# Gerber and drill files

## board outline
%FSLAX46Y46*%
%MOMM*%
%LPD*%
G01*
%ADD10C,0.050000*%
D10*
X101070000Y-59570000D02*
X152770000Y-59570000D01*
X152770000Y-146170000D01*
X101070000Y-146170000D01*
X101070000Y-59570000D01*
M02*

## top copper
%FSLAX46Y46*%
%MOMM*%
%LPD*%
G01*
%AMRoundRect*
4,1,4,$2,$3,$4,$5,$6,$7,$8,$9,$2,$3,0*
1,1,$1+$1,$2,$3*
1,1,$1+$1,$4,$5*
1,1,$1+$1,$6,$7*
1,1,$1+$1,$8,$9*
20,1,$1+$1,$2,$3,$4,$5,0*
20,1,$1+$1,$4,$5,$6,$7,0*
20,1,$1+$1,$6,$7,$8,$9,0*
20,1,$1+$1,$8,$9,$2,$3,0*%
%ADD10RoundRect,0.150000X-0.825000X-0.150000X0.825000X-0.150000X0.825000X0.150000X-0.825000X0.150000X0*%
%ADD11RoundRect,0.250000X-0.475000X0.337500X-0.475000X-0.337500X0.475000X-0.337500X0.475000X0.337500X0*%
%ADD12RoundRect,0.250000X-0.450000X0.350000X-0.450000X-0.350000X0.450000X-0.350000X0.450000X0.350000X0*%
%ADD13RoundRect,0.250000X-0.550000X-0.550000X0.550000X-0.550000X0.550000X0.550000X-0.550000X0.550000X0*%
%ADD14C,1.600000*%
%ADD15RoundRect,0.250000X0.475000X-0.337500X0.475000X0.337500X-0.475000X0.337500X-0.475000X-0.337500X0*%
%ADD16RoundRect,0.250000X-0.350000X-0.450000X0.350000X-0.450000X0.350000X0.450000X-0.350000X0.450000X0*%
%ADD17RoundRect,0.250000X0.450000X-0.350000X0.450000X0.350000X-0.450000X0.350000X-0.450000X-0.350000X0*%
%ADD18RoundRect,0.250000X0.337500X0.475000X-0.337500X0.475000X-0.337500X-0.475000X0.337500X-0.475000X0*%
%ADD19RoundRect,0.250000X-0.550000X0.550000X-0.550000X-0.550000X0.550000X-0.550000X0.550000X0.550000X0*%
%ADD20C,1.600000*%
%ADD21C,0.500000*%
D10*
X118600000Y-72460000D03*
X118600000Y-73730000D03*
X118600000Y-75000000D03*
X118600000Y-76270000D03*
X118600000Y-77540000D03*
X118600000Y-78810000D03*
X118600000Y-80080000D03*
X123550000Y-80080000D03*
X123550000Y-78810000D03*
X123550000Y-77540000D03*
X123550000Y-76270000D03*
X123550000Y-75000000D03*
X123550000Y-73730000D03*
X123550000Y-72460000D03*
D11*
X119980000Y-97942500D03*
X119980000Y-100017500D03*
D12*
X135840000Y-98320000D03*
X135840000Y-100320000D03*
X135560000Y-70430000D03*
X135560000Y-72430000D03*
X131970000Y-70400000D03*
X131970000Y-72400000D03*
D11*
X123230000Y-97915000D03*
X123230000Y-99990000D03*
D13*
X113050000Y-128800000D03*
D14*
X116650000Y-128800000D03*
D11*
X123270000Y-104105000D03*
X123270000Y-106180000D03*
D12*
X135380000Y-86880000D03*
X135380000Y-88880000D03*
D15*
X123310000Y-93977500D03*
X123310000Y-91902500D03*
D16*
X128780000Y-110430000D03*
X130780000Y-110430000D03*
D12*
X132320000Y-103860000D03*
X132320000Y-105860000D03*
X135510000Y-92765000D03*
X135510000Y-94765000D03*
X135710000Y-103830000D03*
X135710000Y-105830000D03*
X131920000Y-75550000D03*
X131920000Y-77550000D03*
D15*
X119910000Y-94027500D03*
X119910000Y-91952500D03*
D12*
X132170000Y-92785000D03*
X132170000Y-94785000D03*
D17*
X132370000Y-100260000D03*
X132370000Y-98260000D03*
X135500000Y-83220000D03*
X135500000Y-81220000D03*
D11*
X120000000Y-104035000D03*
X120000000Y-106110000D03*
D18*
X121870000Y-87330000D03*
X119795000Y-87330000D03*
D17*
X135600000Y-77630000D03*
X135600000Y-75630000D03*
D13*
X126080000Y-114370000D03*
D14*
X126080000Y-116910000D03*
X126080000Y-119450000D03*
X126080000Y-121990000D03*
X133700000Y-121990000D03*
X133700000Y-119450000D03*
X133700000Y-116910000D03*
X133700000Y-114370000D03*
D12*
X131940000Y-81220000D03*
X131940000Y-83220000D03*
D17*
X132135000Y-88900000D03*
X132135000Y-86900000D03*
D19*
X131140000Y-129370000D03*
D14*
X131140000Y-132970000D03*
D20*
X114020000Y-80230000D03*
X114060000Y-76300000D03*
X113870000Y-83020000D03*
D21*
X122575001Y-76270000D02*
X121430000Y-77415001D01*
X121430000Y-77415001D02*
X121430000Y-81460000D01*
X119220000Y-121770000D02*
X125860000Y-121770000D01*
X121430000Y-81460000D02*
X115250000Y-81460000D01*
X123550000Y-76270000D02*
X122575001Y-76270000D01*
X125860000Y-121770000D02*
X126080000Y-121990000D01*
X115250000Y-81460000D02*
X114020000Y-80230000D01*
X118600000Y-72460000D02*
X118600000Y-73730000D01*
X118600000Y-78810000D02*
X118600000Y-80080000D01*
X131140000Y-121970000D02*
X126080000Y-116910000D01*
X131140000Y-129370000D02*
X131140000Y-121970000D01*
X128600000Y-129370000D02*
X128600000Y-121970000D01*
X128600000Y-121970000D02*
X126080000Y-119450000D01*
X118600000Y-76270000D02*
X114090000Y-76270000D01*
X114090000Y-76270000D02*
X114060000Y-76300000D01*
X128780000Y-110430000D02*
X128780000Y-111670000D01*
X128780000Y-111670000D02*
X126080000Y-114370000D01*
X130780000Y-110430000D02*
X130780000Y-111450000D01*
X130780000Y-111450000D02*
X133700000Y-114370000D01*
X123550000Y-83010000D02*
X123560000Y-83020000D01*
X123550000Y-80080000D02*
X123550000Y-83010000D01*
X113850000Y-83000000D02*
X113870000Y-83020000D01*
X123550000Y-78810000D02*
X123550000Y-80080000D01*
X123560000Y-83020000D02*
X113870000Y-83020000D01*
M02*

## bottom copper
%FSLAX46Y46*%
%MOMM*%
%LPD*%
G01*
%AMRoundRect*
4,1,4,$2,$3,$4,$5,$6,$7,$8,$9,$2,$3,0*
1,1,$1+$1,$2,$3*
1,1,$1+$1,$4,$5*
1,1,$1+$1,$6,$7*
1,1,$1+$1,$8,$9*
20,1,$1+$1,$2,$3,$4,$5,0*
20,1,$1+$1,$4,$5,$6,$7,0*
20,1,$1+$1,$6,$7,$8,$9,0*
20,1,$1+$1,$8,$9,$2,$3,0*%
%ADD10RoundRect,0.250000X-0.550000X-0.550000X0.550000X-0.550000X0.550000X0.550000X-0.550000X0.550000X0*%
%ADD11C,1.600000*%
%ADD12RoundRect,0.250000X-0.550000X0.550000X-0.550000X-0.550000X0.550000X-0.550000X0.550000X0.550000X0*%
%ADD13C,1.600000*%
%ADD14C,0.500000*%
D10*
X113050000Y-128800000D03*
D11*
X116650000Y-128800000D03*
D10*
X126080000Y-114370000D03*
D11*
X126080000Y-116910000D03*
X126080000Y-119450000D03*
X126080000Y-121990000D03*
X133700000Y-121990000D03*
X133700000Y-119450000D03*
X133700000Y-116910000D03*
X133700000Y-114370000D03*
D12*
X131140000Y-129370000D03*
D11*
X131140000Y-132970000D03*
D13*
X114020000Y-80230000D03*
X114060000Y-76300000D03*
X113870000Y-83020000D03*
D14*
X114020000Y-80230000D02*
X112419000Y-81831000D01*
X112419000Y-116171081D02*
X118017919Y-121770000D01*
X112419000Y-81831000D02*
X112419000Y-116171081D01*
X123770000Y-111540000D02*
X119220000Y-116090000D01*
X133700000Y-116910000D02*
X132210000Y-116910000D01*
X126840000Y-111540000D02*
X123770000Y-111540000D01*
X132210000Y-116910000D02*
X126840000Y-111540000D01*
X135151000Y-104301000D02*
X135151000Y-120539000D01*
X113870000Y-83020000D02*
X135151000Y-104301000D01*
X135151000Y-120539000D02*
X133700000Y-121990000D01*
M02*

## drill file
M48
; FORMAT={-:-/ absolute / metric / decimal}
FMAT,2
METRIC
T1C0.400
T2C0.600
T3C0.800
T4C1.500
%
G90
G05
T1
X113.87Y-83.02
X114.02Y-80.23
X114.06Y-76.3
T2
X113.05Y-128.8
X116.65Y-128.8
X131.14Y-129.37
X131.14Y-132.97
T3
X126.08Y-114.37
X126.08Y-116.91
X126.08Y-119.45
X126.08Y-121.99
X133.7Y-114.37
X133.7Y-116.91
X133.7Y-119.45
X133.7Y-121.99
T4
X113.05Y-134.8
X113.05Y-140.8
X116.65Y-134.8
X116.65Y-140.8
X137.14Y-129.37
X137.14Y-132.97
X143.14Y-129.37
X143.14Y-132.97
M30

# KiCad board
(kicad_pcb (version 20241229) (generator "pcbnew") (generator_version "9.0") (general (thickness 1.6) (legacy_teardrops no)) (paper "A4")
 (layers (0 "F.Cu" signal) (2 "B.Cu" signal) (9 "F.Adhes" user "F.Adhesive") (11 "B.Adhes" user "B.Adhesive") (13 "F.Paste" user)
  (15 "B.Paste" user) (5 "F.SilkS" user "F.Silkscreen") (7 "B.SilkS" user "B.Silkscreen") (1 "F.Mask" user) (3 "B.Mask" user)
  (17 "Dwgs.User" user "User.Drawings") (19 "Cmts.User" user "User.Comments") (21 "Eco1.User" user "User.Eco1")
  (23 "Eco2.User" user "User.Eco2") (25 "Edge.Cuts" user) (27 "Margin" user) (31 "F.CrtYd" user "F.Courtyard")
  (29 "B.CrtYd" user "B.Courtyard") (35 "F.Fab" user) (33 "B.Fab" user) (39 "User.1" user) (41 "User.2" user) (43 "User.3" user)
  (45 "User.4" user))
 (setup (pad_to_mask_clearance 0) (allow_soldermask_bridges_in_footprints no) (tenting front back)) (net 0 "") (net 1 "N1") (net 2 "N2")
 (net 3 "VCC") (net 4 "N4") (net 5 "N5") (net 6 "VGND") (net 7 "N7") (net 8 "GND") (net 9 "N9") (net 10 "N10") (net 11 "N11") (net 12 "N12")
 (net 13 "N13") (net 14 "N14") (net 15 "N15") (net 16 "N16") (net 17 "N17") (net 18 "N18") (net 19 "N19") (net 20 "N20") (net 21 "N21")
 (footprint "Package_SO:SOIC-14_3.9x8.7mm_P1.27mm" (layer "F.Cu") (at 121.075 76.27)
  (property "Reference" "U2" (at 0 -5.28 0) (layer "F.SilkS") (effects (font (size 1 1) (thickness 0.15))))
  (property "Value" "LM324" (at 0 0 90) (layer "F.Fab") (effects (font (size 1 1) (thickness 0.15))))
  (pad "1" smd roundrect (at -2.475 -3.81) (size 1.95 0.6) (layers "F.Cu" "F.Mask" "F.Paste") (roundrect_rratio 0.25) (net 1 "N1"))
  (pad "2" smd roundrect (at -2.475 -2.54) (size 1.95 0.6) (layers "F.Cu" "F.Mask" "F.Paste") (roundrect_rratio 0.25) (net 1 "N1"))
  (pad "3" smd roundrect (at -2.475 -1.27) (size 1.95 0.6) (layers "F.Cu" "F.Mask" "F.Paste") (roundrect_rratio 0.25) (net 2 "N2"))
  (pad "4" smd roundrect (at -2.475 0) (size 1.95 0.6) (layers "F.Cu" "F.Mask" "F.Paste") (roundrect_rratio 0.25) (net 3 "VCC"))
  (pad "5" smd roundrect (at -2.475 1.27) (size 1.95 0.6) (layers "F.Cu" "F.Mask" "F.Paste") (roundrect_rratio 0.25) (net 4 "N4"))
  (pad "6" smd roundrect (at -2.475 2.54) (size 1.95 0.6) (layers "F.Cu" "F.Mask" "F.Paste") (roundrect_rratio 0.25) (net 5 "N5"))
  (pad "7" smd roundrect (at -2.475 3.81) (size 1.95 0.6) (layers "F.Cu" "F.Mask" "F.Paste") (roundrect_rratio 0.25) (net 5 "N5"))
  (pad "8" smd roundrect (at 2.475 3.81) (size 1.95 0.6) (layers "F.Cu" "F.Mask" "F.Paste") (roundrect_rratio 0.25) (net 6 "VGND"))
  (pad "9" smd roundrect (at 2.475 2.54) (size 1.95 0.6) (layers "F.Cu" "F.Mask" "F.Paste") (roundrect_rratio 0.25) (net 6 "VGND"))
  (pad "10" smd roundrect (at 2.475 1.27) (size 1.95 0.6) (layers "F.Cu" "F.Mask" "F.Paste") (roundrect_rratio 0.25) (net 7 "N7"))
  (pad "11" smd roundrect (at 2.475 0) (size 1.95 0.6) (layers "F.Cu" "F.Mask" "F.Paste") (roundrect_rratio 0.25) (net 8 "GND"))
  (pad "12" smd roundrect (at 2.475 -1.27) (size 1.95 0.6) (layers "F.Cu" "F.Mask" "F.Paste") (roundrect_rratio 0.25) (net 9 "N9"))
  (pad "13" smd roundrect (at 2.475 -2.54) (size 1.95 0.6) (layers "F.Cu" "F.Mask" "F.Paste") (roundrect_rratio 0.25) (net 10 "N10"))
  (pad "14" smd roundrect (at 2.475 -3.81) (size 1.95 0.6) (layers "F.Cu" "F.Mask" "F.Paste") (roundrect_rratio 0.25) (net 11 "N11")))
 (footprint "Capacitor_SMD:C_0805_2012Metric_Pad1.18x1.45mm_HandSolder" (layer "F.Cu") (at 119.98 98.98 -90)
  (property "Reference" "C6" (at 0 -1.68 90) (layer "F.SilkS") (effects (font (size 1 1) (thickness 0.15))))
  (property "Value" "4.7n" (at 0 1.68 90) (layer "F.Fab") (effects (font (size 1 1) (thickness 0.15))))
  (pad "1" smd roundrect (at -1.0375 0 270) (size 1.175 1.45) (layers "F.Cu" "F.Mask" "F.Paste") (roundrect_rratio 0.212766) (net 1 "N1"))
  (pad "2" smd roundrect (at 1.0375 0 270) (size 1.175 1.45) (layers "F.Cu" "F.Mask" "F.Paste") (roundrect_rratio 0.212766) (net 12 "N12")))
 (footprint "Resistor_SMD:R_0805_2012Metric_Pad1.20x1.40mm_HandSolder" (layer "F.Cu") (at 135.84 99.32 -90)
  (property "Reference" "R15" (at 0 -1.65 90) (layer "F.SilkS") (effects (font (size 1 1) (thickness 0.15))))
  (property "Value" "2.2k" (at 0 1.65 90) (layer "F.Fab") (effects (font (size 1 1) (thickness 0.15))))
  (pad "1" smd roundrect (at -1 0 270) (size 1.2 1.4) (layers "F.Cu" "F.Mask" "F.Paste") (roundrect_rratio 0.208333) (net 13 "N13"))
  (pad "2" smd roundrect (at 1 0 270) (size 1.2 1.4) (layers "F.Cu" "F.Mask" "F.Paste") (roundrect_rratio 0.208333) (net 10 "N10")))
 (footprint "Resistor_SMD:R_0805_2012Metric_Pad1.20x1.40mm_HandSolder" (layer "F.Cu") (at 135.56 71.43 -90)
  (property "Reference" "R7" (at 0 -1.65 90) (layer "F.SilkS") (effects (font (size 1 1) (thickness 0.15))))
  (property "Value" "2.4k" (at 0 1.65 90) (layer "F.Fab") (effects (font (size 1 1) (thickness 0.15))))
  (pad "1" smd roundrect (at -1 0 270) (size 1.2 1.4) (layers "F.Cu" "F.Mask" "F.Paste") (roundrect_rratio 0.208333) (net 4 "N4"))
  (pad "2" smd roundrect (at 1 0 270) (size 1.2 1.4) (layers "F.Cu" "F.Mask" "F.Paste") (roundrect_rratio 0.208333) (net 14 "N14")))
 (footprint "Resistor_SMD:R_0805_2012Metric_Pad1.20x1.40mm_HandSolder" (layer "F.Cu") (at 131.97 71.4 -90)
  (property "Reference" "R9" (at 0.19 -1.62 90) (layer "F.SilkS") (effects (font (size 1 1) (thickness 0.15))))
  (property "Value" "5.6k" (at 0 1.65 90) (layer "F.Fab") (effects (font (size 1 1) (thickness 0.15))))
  (pad "1" smd roundrect (at -1 0 270) (size 1.2 1.4) (layers "F.Cu" "F.Mask" "F.Paste") (roundrect_rratio 0.208333) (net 9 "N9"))
  (pad "2" smd roundrect (at 1 0 270) (size 1.2 1.4) (layers "F.Cu" "F.Mask" "F.Paste") (roundrect_rratio 0.208333) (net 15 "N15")))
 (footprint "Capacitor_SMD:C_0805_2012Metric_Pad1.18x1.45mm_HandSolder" (layer "F.Cu") (at 123.23 98.9525 -90)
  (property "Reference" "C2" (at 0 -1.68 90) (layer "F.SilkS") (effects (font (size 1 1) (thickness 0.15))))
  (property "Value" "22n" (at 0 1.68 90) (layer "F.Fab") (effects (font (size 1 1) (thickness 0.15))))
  (pad "1" smd roundrect (at -1.0375 0 270) (size 1.175 1.45) (layers "F.Cu" "F.Mask" "F.Paste") (roundrect_rratio 0.212766) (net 1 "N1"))
  (pad "2" smd roundrect (at 1.0375 0 270) (size 1.175 1.45) (layers "F.Cu" "F.Mask" "F.Paste") (roundrect_rratio 0.212766) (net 12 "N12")))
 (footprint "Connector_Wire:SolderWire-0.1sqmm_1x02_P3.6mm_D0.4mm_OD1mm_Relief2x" (layer "F.Cu") (at 113.05 128.8)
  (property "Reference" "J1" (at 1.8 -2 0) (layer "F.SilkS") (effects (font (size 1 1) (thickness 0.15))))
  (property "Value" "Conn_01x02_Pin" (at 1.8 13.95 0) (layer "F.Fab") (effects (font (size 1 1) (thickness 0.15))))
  (pad "" np_thru_hole circle (at 0 6) (size 1.5 1.5) (drill 1.5) (layers "*.Cu" "*.Mask"))
  (pad "" np_thru_hole circle (at 0 12) (size 1.5 1.5) (drill 1.5) (layers "*.Cu" "*.Mask"))
  (pad "" np_thru_hole circle (at 3.6 6) (size 1.5 1.5) (drill 1.5) (layers "*.Cu" "*.Mask"))
  (pad "" np_thru_hole circle (at 3.6 12) (size 1.5 1.5) (drill 1.5) (layers "*.Cu" "*.Mask"))
  (pad "1" thru_hole roundrect (at 0 0) (size 1.6 1.6) (drill 0.6) (layers "*.Cu" "*.Mask") (remove_unused_layers no)
   (roundrect_rratio 0.15625) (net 3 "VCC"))
  (pad "2" thru_hole circle (at 3.6 0) (size 1.6 1.6) (drill 0.6) (layers "*.Cu" "*.Mask") (remove_unused_layers no) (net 8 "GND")))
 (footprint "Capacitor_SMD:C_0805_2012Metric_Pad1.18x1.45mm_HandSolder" (layer "F.Cu") (at 123.27 105.1425 -90)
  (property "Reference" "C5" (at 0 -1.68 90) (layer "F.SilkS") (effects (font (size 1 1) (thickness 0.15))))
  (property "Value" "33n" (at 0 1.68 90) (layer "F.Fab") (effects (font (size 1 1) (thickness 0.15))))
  (pad "1" smd roundrect (at -1.0375 0 270) (size 1.175 1.45) (layers "F.Cu" "F.Mask" "F.Paste") (roundrect_rratio 0.212766) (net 5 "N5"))
  (pad "2" smd roundrect (at 1.0375 0 270) (size 1.175 1.45) (layers "F.Cu" "F.Mask" "F.Paste") (roundrect_rratio 0.212766) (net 14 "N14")))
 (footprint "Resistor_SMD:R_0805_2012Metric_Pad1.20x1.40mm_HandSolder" (layer "F.Cu") (at 135.38 87.88 -90)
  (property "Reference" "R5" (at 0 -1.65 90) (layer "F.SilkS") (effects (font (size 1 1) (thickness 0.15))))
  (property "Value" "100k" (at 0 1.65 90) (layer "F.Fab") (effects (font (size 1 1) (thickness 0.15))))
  (pad "1" smd roundrect (at -1 0 270) (size 1.2 1.4) (layers "F.Cu" "F.Mask" "F.Paste") (roundrect_rratio 0.208333) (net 7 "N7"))
  (pad "2" smd roundrect (at 1 0 270) (size 1.2 1.4) (layers "F.Cu" "F.Mask" "F.Paste") (roundrect_rratio 0.208333) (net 8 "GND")))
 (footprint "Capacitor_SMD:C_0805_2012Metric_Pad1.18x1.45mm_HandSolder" (layer "F.Cu") (at 123.31 92.94 90)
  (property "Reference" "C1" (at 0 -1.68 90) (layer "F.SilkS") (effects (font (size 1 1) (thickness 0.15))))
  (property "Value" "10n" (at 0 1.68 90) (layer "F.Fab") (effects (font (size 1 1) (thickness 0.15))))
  (pad "1" smd roundrect (at -1.0375 0 90) (size 1.175 1.45) (layers "F.Cu" "F.Mask" "F.Paste") (roundrect_rratio 0.212766) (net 2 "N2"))
  (pad "2" smd roundrect (at 1.0375 0 90) (size 1.175 1.45) (layers "F.Cu" "F.Mask" "F.Paste") (roundrect_rratio 0.212766) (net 8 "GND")))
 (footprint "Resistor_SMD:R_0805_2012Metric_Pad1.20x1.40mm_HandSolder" (layer "F.Cu") (at 129.78 110.43)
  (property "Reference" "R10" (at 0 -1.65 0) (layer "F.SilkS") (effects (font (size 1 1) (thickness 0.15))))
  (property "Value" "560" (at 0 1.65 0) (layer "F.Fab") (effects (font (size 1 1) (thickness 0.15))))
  (pad "1" smd roundrect (at -1 0) (size 1.2 1.4) (layers "F.Cu" "F.Mask" "F.Paste") (roundrect_rratio 0.208333) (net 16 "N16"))
  (pad "2" smd roundrect (at 1 0) (size 1.2 1.4) (layers "F.Cu" "F.Mask" "F.Paste") (roundrect_rratio 0.208333) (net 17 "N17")))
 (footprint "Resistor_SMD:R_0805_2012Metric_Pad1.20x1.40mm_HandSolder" (layer "F.Cu") (at 132.32 104.86 -90)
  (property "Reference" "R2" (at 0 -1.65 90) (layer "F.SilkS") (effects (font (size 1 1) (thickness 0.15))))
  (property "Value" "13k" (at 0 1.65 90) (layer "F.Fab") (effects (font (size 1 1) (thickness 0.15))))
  (pad "1" smd roundrect (at -1 0 270) (size 1.2 1.4) (layers "F.Cu" "F.Mask" "F.Paste") (roundrect_rratio 0.208333) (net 12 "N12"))
  (pad "2" smd roundrect (at 1 0 270) (size 1.2 1.4) (layers "F.Cu" "F.Mask" "F.Paste") (roundrect_rratio 0.208333) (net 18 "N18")))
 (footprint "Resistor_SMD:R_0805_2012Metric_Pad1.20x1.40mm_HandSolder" (layer "F.Cu") (at 135.51 93.765 -90)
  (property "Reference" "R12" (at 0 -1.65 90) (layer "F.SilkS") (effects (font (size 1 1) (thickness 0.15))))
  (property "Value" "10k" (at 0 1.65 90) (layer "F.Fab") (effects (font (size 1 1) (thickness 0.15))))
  (pad "1" smd roundrect (at -1 0 270) (size 1.2 1.4) (layers "F.Cu" "F.Mask" "F.Paste") (roundrect_rratio 0.208333) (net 10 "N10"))
  (pad "2" smd roundrect (at 1 0 270) (size 1.2 1.4) (layers "F.Cu" "F.Mask" "F.Paste") (roundrect_rratio 0.208333) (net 8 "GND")))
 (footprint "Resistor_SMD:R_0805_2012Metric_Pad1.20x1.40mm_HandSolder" (layer "F.Cu") (at 135.71 104.83 -90)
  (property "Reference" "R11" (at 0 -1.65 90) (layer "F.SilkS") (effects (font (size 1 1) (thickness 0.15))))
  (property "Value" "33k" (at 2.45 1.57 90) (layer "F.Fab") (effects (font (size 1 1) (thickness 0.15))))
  (pad "1" smd roundrect (at -1 0 270) (size 1.2 1.4) (layers "F.Cu" "F.Mask" "F.Paste") (roundrect_rratio 0.208333) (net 3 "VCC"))
  (pad "2" smd roundrect (at 1 0 270) (size 1.2 1.4) (layers "F.Cu" "F.Mask" "F.Paste") (roundrect_rratio 0.208333) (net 10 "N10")))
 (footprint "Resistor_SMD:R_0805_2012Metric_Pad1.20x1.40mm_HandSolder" (layer "F.Cu") (at 131.92 76.55 -90)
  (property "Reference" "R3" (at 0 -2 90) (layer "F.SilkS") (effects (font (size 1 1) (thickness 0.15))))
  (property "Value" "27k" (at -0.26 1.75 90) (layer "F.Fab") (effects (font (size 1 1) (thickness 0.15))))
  (pad "1" smd roundrect (at -1 0 270) (size 1.2 1.4) (layers "F.Cu" "F.Mask" "F.Paste") (roundrect_rratio 0.208333) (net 2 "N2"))
  (pad "2" smd roundrect (at 1 0 270) (size 1.2 1.4) (layers "F.Cu" "F.Mask" "F.Paste") (roundrect_rratio 0.208333) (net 12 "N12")))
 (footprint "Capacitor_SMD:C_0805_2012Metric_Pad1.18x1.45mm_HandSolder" (layer "F.Cu") (at 119.91 92.99 90)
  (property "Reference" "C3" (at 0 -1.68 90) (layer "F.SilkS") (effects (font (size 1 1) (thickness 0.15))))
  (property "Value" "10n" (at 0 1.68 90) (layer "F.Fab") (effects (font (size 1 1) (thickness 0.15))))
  (pad "1" smd roundrect (at -1.0375 0 90) (size 1.175 1.45) (layers "F.Cu" "F.Mask" "F.Paste") (roundrect_rratio 0.212766) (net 4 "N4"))
  (pad "2" smd roundrect (at 1.0375 0 90) (size 1.175 1.45) (layers "F.Cu" "F.Mask" "F.Paste") (roundrect_rratio 0.212766) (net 8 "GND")))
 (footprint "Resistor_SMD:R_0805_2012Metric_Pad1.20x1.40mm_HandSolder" (layer "F.Cu") (at 132.17 93.785 -90)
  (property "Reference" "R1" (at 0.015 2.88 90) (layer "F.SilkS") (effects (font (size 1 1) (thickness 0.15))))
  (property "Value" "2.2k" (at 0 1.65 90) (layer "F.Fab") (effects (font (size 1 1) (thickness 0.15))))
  (pad "1" smd roundrect (at -1 0 270) (size 1.2 1.4) (layers "F.Cu" "F.Mask" "F.Paste") (roundrect_rratio 0.208333) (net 15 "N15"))
  (pad "2" smd roundrect (at 1 0 270) (size 1.2 1.4) (layers "F.Cu" "F.Mask" "F.Paste") (roundrect_rratio 0.208333) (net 8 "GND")))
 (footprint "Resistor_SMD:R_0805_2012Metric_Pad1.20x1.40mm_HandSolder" (layer "F.Cu") (at 132.37 99.26 90)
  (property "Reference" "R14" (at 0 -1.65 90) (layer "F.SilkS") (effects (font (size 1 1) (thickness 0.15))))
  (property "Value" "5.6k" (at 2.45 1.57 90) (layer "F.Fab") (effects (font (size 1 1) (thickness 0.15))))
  (pad "1" smd roundrect (at -1 0 90) (size 1.2 1.4) (layers "F.Cu" "F.Mask" "F.Paste") (roundrect_rratio 0.208333) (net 11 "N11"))
  (pad "2" smd roundrect (at 1 0 90) (size 1.2 1.4) (layers "F.Cu" "F.Mask" "F.Paste") (roundrect_rratio 0.208333) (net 13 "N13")))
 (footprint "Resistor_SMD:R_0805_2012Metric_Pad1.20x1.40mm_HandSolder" (layer "F.Cu") (at 135.5 82.22 90)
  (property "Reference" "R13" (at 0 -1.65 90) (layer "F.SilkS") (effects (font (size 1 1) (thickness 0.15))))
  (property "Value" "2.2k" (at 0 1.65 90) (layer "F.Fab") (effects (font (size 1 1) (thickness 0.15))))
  (pad "1" smd roundrect (at -1 0 90) (size 1.2 1.4) (layers "F.Cu" "F.Mask" "F.Paste") (roundrect_rratio 0.208333) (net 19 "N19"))
  (pad "2" smd roundrect (at 1 0 90) (size 1.2 1.4) (layers "F.Cu" "F.Mask" "F.Paste") (roundrect_rratio 0.208333) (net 9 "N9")))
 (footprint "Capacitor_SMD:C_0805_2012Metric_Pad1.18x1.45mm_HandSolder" (layer "F.Cu") (at 120 105.0725 -90)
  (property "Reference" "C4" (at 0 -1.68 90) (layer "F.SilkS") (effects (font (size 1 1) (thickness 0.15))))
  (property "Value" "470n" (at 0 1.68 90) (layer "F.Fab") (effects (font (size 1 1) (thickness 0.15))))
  (pad "1" smd roundrect (at -1.0375 0 270) (size 1.175 1.45) (layers "F.Cu" "F.Mask" "F.Paste") (roundrect_rratio 0.212766) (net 5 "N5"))
  (pad "2" smd roundrect (at 1.0375 0 270) (size 1.175 1.45) (layers "F.Cu" "F.Mask" "F.Paste") (roundrect_rratio 0.212766) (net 14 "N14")))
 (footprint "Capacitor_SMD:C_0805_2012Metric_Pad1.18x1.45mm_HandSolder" (layer "F.Cu") (at 120.8325 87.33 180)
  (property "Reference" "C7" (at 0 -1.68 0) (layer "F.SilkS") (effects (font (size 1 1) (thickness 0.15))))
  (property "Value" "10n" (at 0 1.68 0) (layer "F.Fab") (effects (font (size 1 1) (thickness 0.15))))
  (pad "1" smd roundrect (at -1.0375 0 180) (size 1.175 1.45) (layers "F.Cu" "F.Mask" "F.Paste") (roundrect_rratio 0.212766) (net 3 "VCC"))
  (pad "2" smd roundrect (at 1.0375 0 180) (size 1.175 1.45) (layers "F.Cu" "F.Mask" "F.Paste") (roundrect_rratio 0.212766) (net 8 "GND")))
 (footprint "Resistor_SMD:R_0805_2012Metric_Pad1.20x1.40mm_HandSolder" (layer "F.Cu") (at 135.6 76.63 90)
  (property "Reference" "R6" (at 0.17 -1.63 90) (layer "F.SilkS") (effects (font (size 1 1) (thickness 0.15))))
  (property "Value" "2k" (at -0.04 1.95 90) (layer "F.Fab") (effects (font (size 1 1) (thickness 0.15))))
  (pad "1" smd roundrect (at -1 0 90) (size 1.2 1.4) (layers "F.Cu" "F.Mask" "F.Paste") (roundrect_rratio 0.208333) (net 14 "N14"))
  (pad "2" smd roundrect (at 1 0 90) (size 1.2 1.4) (layers "F.Cu" "F.Mask" "F.Paste") (roundrect_rratio 0.208333) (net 1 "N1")))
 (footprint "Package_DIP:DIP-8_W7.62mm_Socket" (layer "F.Cu") (at 126.08 114.37)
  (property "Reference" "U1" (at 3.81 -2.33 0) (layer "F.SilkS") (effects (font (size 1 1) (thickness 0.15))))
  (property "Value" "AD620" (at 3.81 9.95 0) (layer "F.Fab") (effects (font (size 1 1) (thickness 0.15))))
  (pad "1" thru_hole roundrect (at 0 0) (size 1.6 1.6) (drill 0.8) (layers "*.Cu" "*.Mask") (remove_unused_layers no)
   (roundrect_rratio 0.15625) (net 16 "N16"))
  (pad "2" thru_hole circle (at 0 2.54) (size 1.6 1.6) (drill 0.8) (layers "*.Cu" "*.Mask") (remove_unused_layers no) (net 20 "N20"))
  (pad "3" thru_hole circle (at 0 5.08) (size 1.6 1.6) (drill 0.8) (layers "*.Cu" "*.Mask") (remove_unused_layers no) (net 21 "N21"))
  (pad "4" thru_hole circle (at 0 7.62) (size 1.6 1.6) (drill 0.8) (layers "*.Cu" "*.Mask") (remove_unused_layers no) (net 8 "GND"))
  (pad "5" thru_hole circle (at 7.62 7.62) (size 1.6 1.6) (drill 0.8) (layers "*.Cu" "*.Mask") (remove_unused_layers no) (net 6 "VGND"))
  (pad "6" thru_hole circle (at 7.62 5.08) (size 1.6 1.6) (drill 0.8) (layers "*.Cu" "*.Mask") (remove_unused_layers no) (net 18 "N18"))
  (pad "7" thru_hole circle (at 7.62 2.54) (size 1.6 1.6) (drill 0.8) (layers "*.Cu" "*.Mask") (remove_unused_layers no) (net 3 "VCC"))
  (pad "8" thru_hole circle (at 7.62 0) (size 1.6 1.6) (drill 0.8) (layers "*.Cu" "*.Mask") (remove_unused_layers no) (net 17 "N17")))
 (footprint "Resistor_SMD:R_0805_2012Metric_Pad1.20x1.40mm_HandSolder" (layer "F.Cu") (at 131.94 82.22 -90)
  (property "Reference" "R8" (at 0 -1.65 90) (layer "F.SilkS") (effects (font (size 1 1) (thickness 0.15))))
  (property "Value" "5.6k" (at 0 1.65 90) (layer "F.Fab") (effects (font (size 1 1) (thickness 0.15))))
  (pad "1" smd roundrect (at -1 0 270) (size 1.2 1.4) (layers "F.Cu" "F.Mask" "F.Paste") (roundrect_rratio 0.208333) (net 5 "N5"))
  (pad "2" smd roundrect (at 1 0 270) (size 1.2 1.4) (layers "F.Cu" "F.Mask" "F.Paste") (roundrect_rratio 0.208333) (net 19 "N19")))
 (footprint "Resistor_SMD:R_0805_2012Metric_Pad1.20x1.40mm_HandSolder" (layer "F.Cu") (at 132.135 87.9 90)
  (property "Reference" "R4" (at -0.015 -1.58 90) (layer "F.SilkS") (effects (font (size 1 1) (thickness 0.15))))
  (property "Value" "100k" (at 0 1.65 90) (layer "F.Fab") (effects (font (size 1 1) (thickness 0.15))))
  (pad "1" smd roundrect (at -1 0 90) (size 1.2 1.4) (layers "F.Cu" "F.Mask" "F.Paste") (roundrect_rratio 0.208333) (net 3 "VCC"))
  (pad "2" smd roundrect (at 1 0 90) (size 1.2 1.4) (layers "F.Cu" "F.Mask" "F.Paste") (roundrect_rratio 0.208333) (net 7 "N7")))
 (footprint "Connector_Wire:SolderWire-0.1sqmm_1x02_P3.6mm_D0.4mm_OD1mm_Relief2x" (layer "B.Cu") (at 131.14 129.37 -90)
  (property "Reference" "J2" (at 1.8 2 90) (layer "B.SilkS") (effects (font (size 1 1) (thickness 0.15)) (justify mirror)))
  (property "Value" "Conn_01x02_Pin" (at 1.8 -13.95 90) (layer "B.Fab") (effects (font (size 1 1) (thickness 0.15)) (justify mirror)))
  (pad "" np_thru_hole circle (at 0 -12 270) (size 1.5 1.5) (drill 1.5) (layers "*.Cu" "*.Mask"))
  (pad "" np_thru_hole circle (at 0 -6 270) (size 1.5 1.5) (drill 1.5) (layers "*.Cu" "*.Mask"))
  (pad "" np_thru_hole circle (at 3.6 -12 270) (size 1.5 1.5) (drill 1.5) (layers "*.Cu" "*.Mask"))
  (pad "" np_thru_hole circle (at 3.6 -6 270) (size 1.5 1.5) (drill 1.5) (layers "*.Cu" "*.Mask"))
  (pad "1" thru_hole roundrect (at 0 0 270) (size 1.6 1.6) (drill 0.6) (layers "*.Cu" "*.Mask") (remove_unused_layers no)
   (roundrect_rratio 0.15625) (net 20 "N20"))
  (pad "2" thru_hole circle (at 3.6 0 270) (size 1.6 1.6) (drill 0.6) (layers "*.Cu" "*.Mask") (remove_unused_layers no) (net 21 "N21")))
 (gr_rect (start 101.07 59.57) (end 152.77 146.17) (stroke (width 0.05) (type default)) (fill no) (layer "Edge.Cuts"))
 (segment (start 122.575001 76.27) (end 121.43 77.415001) (width 0.5) (layer "F.Cu") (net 8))
 (segment (start 121.43 77.415001) (end 121.43 81.46) (width 0.5) (layer "F.Cu") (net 8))
 (segment (start 119.22 121.77) (end 125.86 121.77) (width 0.5) (layer "F.Cu") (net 8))
 (segment (start 121.43 81.46) (end 115.25 81.46) (width 0.5) (layer "F.Cu") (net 8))
 (segment (start 123.55 76.27) (end 122.575001 76.27) (width 0.5) (layer "F.Cu") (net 8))
 (segment (start 125.86 121.77) (end 126.08 121.99) (width 0.5) (layer "F.Cu") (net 8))
 (segment (start 115.25 81.46) (end 114.02 80.23) (width 0.5) (layer "F.Cu") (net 8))
 (via (at 114.02 80.23) (size 1.6) (drill 0.4) (layers "F.Cu" "B.Cu") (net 8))
 (segment (start 114.02 80.23) (end 112.419 81.831) (width 0.5) (layer "B.Cu") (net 8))
 (segment (start 112.419 116.171081) (end 118.017919 121.77) (width 0.5) (layer "B.Cu") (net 8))
 (segment (start 112.419 81.831) (end 112.419 116.171081) (width 0.5) (layer "B.Cu") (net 8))
 (segment (start 118.6 72.46) (end 118.6 73.73) (width 0.5) (layer "F.Cu") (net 1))
 (segment (start 118.6 78.81) (end 118.6 80.08) (width 0.5) (layer "F.Cu") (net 5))
 (segment (start 131.14 121.97) (end 126.08 116.91) (width 0.5) (layer "F.Cu") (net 20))
 (segment (start 131.14 129.37) (end 131.14 121.97) (width 0.5) (layer "F.Cu") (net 20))
 (segment (start 128.6 129.37) (end 128.6 121.97) (width 0.5) (layer "F.Cu") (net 21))
 (segment (start 128.6 121.97) (end 126.08 119.45) (width 0.5) (layer "F.Cu") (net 21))
 (segment (start 118.6 76.27) (end 114.09 76.27) (width 0.5) (layer "F.Cu") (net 3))
 (segment (start 114.09 76.27) (end 114.06 76.3) (width 0.5) (layer "F.Cu") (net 3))
 (via (at 114.06 76.3) (size 1.6) (drill 0.4) (layers "F.Cu" "B.Cu") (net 3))
 (segment (start 123.77 111.54) (end 119.22 116.09) (width 0.5) (layer "B.Cu") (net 3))
 (segment (start 133.7 116.91) (end 132.21 116.91) (width 0.5) (layer "B.Cu") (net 3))
 (segment (start 126.84 111.54) (end 123.77 111.54) (width 0.5) (layer "B.Cu") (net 3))
 (segment (start 132.21 116.91) (end 126.84 111.54) (width 0.5) (layer "B.Cu") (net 3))
 (segment (start 128.78 110.43) (end 128.78 111.67) (width 0.5) (layer "F.Cu") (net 16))
 (segment (start 128.78 111.67) (end 126.08 114.37) (width 0.5) (layer "F.Cu") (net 16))
 (segment (start 130.78 110.43) (end 130.78 111.45) (width 0.5) (layer "F.Cu") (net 17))
 (segment (start 130.78 111.45) (end 133.7 114.37) (width 0.5) (layer "F.Cu") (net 17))
 (segment (start 123.55 83.01) (end 123.56 83.02) (width 0.5) (layer "F.Cu") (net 6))
 (segment (start 123.55 80.08) (end 123.55 83.01) (width 0.5) (layer "F.Cu") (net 6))
 (segment (start 113.85 83) (end 113.87 83.02) (width 0.5) (layer "F.Cu") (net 6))
 (segment (start 123.55 78.81) (end 123.55 80.08) (width 0.5) (layer "F.Cu") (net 6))
 (segment (start 123.56 83.02) (end 113.87 83.02) (width 0.5) (layer "F.Cu") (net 6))
 (via (at 113.87 83.02) (size 1.6) (drill 0.4) (layers "F.Cu" "B.Cu") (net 6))
 (segment (start 135.151 104.301) (end 135.151 120.539) (width 0.5) (layer "B.Cu") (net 6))
 (segment (start 113.87 83.02) (end 135.151 104.301) (width 0.5) (layer "B.Cu") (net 6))
 (segment (start 135.151 120.539) (end 133.7 121.99) (width 0.5) (layer "B.Cu") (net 6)))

